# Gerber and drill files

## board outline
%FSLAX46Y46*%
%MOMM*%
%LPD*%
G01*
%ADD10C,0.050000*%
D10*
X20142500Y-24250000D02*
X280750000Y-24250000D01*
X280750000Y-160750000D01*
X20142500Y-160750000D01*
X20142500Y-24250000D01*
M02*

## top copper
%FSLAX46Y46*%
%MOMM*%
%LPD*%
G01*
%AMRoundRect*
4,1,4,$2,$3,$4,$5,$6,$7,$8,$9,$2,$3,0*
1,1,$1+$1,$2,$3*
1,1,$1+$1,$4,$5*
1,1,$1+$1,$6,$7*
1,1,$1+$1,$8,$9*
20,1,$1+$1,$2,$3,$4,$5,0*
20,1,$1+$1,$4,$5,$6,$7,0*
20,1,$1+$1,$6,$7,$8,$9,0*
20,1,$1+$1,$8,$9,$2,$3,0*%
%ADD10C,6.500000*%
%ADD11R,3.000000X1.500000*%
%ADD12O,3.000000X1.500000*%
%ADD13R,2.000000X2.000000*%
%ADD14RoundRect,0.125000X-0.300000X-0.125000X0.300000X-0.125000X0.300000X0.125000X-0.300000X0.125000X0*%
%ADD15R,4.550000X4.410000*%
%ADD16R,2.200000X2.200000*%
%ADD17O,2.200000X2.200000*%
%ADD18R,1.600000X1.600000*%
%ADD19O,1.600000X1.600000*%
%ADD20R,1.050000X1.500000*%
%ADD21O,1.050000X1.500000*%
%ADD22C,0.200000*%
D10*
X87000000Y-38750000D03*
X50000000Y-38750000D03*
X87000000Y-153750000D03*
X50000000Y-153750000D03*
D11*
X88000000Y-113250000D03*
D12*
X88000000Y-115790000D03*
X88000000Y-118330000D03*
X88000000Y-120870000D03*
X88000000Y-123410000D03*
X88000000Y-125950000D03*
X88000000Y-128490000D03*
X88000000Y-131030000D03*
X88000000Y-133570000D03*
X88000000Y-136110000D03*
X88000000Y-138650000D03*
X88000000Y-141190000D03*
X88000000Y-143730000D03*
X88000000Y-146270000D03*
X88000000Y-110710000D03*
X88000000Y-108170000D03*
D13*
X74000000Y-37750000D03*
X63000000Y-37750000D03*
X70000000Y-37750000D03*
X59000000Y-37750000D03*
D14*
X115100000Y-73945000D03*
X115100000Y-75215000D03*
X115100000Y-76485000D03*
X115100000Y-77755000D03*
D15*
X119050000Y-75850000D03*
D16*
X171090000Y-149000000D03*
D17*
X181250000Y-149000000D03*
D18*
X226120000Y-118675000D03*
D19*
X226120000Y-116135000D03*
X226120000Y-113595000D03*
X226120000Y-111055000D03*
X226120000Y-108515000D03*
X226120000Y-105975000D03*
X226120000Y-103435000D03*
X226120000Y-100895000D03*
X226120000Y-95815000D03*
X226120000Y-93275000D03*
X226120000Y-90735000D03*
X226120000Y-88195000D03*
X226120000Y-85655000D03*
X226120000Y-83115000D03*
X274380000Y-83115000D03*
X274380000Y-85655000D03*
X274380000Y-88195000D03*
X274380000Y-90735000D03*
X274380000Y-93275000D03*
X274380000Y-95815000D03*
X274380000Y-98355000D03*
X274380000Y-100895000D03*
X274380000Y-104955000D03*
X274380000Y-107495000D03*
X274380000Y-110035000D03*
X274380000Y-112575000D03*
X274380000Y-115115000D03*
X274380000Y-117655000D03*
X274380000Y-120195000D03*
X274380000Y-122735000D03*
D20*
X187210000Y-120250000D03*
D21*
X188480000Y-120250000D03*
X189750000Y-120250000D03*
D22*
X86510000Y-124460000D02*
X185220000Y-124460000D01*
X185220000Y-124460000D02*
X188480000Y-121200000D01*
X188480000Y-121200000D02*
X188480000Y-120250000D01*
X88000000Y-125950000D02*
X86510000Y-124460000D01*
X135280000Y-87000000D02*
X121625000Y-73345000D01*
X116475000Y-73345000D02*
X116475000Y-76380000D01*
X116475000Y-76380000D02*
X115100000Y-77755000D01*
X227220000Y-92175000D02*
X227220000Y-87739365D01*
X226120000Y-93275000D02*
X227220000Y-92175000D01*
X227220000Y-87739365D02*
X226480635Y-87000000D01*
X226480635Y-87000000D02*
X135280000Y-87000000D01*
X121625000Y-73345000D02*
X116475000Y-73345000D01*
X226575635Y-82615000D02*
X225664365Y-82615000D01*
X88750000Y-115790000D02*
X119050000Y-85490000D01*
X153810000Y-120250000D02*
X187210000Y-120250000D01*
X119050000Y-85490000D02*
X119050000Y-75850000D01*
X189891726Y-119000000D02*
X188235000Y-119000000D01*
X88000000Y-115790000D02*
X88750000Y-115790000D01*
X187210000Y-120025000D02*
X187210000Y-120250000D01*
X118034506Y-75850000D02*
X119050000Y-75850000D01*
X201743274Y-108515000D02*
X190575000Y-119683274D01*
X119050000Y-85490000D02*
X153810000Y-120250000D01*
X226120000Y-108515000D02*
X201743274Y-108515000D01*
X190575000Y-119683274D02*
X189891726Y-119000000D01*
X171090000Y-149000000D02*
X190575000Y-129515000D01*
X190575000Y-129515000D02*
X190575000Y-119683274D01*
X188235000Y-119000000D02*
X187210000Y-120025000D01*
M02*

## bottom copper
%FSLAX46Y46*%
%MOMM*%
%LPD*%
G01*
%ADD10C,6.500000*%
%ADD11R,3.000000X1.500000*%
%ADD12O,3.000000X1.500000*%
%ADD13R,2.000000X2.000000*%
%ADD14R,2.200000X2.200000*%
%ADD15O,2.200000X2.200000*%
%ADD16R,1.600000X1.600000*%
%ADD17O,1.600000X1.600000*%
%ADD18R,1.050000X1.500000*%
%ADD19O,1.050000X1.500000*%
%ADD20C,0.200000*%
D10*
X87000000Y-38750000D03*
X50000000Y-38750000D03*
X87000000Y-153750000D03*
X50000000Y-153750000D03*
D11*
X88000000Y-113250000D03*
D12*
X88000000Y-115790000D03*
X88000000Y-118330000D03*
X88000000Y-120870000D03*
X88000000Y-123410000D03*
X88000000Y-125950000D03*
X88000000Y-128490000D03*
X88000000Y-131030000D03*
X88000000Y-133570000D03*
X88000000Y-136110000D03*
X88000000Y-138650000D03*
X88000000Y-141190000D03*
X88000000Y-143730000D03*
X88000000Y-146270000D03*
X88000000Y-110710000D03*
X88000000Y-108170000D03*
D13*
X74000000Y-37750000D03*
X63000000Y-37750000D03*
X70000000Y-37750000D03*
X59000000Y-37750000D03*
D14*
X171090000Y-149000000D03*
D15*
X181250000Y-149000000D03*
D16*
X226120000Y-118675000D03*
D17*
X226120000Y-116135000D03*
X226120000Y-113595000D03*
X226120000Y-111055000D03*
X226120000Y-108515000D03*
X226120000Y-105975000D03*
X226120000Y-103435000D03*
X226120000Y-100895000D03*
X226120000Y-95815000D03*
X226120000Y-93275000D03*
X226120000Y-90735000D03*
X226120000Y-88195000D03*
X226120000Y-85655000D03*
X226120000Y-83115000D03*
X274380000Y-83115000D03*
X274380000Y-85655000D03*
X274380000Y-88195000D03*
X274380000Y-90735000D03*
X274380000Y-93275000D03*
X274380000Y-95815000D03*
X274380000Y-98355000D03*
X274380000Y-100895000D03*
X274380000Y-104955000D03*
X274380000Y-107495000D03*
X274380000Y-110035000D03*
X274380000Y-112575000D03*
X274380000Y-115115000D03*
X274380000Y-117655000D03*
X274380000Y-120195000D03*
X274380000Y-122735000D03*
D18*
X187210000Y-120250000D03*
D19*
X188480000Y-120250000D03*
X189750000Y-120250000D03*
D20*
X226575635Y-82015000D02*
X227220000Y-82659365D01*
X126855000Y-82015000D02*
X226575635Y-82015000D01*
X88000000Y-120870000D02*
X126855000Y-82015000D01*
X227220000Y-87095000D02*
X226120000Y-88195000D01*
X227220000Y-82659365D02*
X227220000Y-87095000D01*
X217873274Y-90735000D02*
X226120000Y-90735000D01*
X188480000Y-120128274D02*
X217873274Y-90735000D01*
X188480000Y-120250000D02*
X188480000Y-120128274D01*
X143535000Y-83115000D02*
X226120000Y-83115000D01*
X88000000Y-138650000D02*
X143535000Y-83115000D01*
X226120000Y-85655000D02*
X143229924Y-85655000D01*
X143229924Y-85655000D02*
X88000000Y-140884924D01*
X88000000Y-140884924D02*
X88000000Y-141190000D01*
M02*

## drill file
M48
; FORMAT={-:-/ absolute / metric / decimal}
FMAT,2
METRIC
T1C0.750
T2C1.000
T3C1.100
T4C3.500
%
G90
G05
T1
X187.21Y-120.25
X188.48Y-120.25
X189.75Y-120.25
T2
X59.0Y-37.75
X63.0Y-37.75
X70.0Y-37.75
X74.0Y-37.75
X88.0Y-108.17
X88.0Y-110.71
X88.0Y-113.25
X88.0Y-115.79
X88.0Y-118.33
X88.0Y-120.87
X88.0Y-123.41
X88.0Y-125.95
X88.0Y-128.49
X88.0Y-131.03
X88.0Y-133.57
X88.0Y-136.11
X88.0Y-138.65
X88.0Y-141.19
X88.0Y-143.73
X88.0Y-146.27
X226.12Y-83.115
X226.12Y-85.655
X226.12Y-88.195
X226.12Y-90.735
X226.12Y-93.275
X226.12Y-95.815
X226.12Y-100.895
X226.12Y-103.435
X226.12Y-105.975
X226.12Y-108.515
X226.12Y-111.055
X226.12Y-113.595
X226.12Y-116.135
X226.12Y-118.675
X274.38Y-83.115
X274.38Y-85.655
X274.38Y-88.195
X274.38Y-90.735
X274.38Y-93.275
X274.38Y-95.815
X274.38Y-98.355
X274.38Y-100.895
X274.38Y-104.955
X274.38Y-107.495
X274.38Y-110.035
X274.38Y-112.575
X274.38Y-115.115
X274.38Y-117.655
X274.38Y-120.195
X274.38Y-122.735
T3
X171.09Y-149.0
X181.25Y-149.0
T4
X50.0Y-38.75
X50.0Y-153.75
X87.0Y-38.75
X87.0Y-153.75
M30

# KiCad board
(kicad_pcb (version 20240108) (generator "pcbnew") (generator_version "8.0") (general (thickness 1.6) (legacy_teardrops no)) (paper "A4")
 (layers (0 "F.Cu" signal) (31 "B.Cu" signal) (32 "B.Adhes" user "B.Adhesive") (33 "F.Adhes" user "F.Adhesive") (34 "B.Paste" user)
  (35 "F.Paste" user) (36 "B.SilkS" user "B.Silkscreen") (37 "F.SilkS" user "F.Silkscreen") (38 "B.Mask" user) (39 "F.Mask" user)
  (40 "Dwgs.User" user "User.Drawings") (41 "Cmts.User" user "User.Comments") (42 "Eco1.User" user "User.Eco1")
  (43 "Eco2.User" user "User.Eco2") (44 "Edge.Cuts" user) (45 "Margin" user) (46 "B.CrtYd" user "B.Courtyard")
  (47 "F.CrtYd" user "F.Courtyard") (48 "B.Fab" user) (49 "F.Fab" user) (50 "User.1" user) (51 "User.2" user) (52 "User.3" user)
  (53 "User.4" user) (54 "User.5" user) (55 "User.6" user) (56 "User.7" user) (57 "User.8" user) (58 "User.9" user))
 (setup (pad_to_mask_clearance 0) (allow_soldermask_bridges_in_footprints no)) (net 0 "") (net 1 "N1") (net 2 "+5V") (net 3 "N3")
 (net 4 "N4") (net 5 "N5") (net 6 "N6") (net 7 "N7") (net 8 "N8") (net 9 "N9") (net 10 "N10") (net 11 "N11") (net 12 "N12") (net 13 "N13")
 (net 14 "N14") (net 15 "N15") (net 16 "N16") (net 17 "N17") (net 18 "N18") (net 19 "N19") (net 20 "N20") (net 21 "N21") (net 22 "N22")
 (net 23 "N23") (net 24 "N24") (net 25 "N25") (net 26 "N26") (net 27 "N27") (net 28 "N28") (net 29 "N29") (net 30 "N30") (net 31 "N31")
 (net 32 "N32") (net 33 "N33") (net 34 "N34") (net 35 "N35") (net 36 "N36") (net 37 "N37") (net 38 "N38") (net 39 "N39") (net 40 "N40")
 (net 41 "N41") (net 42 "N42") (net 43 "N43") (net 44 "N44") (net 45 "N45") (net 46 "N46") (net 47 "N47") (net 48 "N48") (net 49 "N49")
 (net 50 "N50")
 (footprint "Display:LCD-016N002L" (layer "F.Cu") (at 88 113.25 -90)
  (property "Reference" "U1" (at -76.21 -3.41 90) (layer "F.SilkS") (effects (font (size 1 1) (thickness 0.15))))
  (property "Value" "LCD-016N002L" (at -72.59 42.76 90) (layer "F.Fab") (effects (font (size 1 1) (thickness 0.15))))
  (pad "" thru_hole circle (at -74.5 1 90) (size 6.5 6.5) (drill 3.5) (layers "*.Cu" "*.Mask") (remove_unused_layers no))
  (pad "" thru_hole circle (at -74.5 38 90) (size 6.5 6.5) (drill 3.5) (layers "*.Cu" "*.Mask") (remove_unused_layers no))
  (pad "" thru_hole circle (at 40.5 1 90) (size 6.5 6.5) (drill 3.5) (layers "*.Cu" "*.Mask") (remove_unused_layers no))
  (pad "" thru_hole circle (at 40.5 38 90) (size 6.5 6.5) (drill 3.5) (layers "*.Cu" "*.Mask") (remove_unused_layers no))
  (pad "1" thru_hole rect (at 0 0 90) (size 1.5 3) (drill 1) (layers "*.Cu" "*.Mask") (remove_unused_layers no) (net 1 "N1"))
  (pad "2" thru_hole oval (at 2.54 0 90) (size 1.5 3) (drill 1) (layers "*.Cu" "*.Mask") (remove_unused_layers no) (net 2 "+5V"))
  (pad "3" thru_hole oval (at 5.08 0 90) (size 1.5 3) (drill 1) (layers "*.Cu" "*.Mask") (remove_unused_layers no) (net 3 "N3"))
  (pad "4" thru_hole oval (at 7.62 0 90) (size 1.5 3) (drill 1) (layers "*.Cu" "*.Mask") (remove_unused_layers no) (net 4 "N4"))
  (pad "5" thru_hole oval (at 10.16 0 90) (size 1.5 3) (drill 1) (layers "*.Cu" "*.Mask") (remove_unused_layers no) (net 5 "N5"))
  (pad "6" thru_hole oval (at 12.7 0 90) (size 1.5 3) (drill 1) (layers "*.Cu" "*.Mask") (remove_unused_layers no) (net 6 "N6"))
  (pad "7" thru_hole oval (at 15.24 0 90) (size 1.5 3) (drill 1) (layers "*.Cu" "*.Mask") (remove_unused_layers no) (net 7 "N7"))
  (pad "8" thru_hole oval (at 17.78 0 90) (size 1.5 3) (drill 1) (layers "*.Cu" "*.Mask") (remove_unused_layers no) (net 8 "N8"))
  (pad "9" thru_hole oval (at 20.32 0 90) (size 1.5 3) (drill 1) (layers "*.Cu" "*.Mask") (remove_unused_layers no) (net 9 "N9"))
  (pad "10" thru_hole oval (at 22.86 0 90) (size 1.5 3) (drill 1) (layers "*.Cu" "*.Mask") (remove_unused_layers no) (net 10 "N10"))
  (pad "11" thru_hole oval (at 25.4 0 90) (size 1.5 3) (drill 1) (layers "*.Cu" "*.Mask") (remove_unused_layers no) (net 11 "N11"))
  (pad "12" thru_hole oval (at 27.94 0 90) (size 1.5 3) (drill 1) (layers "*.Cu" "*.Mask") (remove_unused_layers no) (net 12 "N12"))
  (pad "13" thru_hole oval (at 30.48 0 90) (size 1.5 3) (drill 1) (layers "*.Cu" "*.Mask") (remove_unused_layers no) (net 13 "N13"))
  (pad "14" thru_hole oval (at 33.02 0 90) (size 1.5 3) (drill 1) (layers "*.Cu" "*.Mask") (remove_unused_layers no) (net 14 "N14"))
  (pad "15" thru_hole oval (at -2.54 0 90) (size 1.5 3) (drill 1) (layers "*.Cu" "*.Mask") (remove_unused_layers no) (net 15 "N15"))
  (pad "16" thru_hole oval (at -5.08 0 90) (size 1.5 3) (drill 1) (layers "*.Cu" "*.Mask") (remove_unused_layers no) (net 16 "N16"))
  (pad "A1" thru_hole rect (at -75.5 14 90) (size 2 2) (drill 1) (layers "*.Cu" "*.Mask") (remove_unused_layers no) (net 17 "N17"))
  (pad "A2" thru_hole rect (at -75.5 25 90) (size 2 2) (drill 1) (layers "*.Cu" "*.Mask") (remove_unused_layers no) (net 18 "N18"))
  (pad "K1" thru_hole rect (at -75.5 18 90) (size 2 2) (drill 1) (layers "*.Cu" "*.Mask") (remove_unused_layers no) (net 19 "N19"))
  (pad "K2" thru_hole rect (at -75.5 29 90) (size 2 2) (drill 1) (layers "*.Cu" "*.Mask") (remove_unused_layers no) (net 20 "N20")))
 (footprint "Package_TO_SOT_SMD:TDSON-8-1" (layer "F.Cu") (at 118 75.85)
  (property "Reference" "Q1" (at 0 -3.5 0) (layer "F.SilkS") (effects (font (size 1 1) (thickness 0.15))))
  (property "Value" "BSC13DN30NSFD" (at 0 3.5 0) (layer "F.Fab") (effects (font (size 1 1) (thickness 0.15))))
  (pad "" smd roundrect (at -0.2 -0.85) (size 1.5 1.5) (layers "F.Paste") (roundrect_rratio 0.25))
  (pad "" smd roundrect (at -0.2 0.85) (size 1.5 1.5) (layers "F.Paste") (roundrect_rratio 0.25))
  (pad "" smd custom (at 0.65 0) (size 3.75 4.41) (layers "F.Mask") (zone_connect 0) (thermal_bridge_angle 45)
   (options (clearance outline) (anchor rect)) (primitives))
  (pad "" smd roundrect (at 1.5 -0.85) (size 1.5 1.5) (layers "F.Paste") (roundrect_rratio 0.25))
  (pad "" smd roundrect (at 1.5 0.85) (size 1.5 1.5) (layers "F.Paste") (roundrect_rratio 0.25))
  (pad "" smd roundrect (at 2.905 -1.905) (size 0.75 0.5) (layers "F.Paste") (roundrect_rratio 0.25))
  (pad "" smd roundrect (at 2.905 -0.635) (size 0.75 0.5) (layers "F.Paste") (roundrect_rratio 0.25))
  (pad "" smd roundrect (at 2.905 0.635) (size 0.75 0.5) (layers "F.Paste") (roundrect_rratio 0.25))
  (pad "" smd roundrect (at 2.905 1.905) (size 0.75 0.5) (layers "F.Paste") (roundrect_rratio 0.25))
  (pad "1" smd roundrect (at -2.9 -1.905) (size 0.85 0.5) (layers "F.Cu" "F.Paste" "F.Mask") (roundrect_rratio 0.25) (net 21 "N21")
   (solder_paste_margin -0.05))
  (pad "2" smd roundrect (at -2.9 -0.635) (size 0.85 0.5) (layers "F.Cu" "F.Paste" "F.Mask") (roundrect_rratio 0.25) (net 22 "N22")
   (solder_paste_margin -0.05))
  (pad "3" smd roundrect (at -2.9 0.635) (size 0.85 0.5) (layers "F.Cu" "F.Paste" "F.Mask") (roundrect_rratio 0.25) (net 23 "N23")
   (solder_paste_margin -0.05))
  (pad "4" smd roundrect (at -2.9 1.905) (size 0.85 0.5) (layers "F.Cu" "F.Paste" "F.Mask") (roundrect_rratio 0.25) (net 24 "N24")
   (solder_paste_margin -0.05))
  (pad "5" smd rect (at 1.05 0) (size 4.55 4.41) (layers "F.Cu") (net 2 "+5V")))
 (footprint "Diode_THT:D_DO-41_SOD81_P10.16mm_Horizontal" (layer "F.Cu") (at 171.09 149)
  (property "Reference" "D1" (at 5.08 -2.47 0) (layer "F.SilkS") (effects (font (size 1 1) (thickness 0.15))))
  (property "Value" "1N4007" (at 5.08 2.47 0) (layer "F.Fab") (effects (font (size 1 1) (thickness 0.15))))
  (pad "1" thru_hole rect (at 0 0) (size 2.2 2.2) (drill 1.1) (layers "*.Cu" "*.Mask") (remove_unused_layers no) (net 2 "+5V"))
  (pad "2" thru_hole oval (at 10.16 0) (size 2.2 2.2) (drill 1.1) (layers "*.Cu" "*.Mask") (remove_unused_layers no) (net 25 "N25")))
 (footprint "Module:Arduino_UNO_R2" (layer "F.Cu") (at 226.12 118.675 90)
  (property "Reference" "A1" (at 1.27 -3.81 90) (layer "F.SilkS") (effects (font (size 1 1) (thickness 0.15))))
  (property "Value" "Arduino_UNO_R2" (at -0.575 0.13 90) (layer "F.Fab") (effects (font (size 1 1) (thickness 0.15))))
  (pad "1" thru_hole rect (at 0 0 180) (size 1.6 1.6) (drill 1) (layers "*.Cu" "*.Mask") (remove_unused_layers no) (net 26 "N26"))
  (pad "2" thru_hole oval (at 2.54 0 180) (size 1.6 1.6) (drill 1) (layers "*.Cu" "*.Mask") (remove_unused_layers no) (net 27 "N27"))
  (pad "3" thru_hole oval (at 5.08 0 180) (size 1.6 1.6) (drill 1) (layers "*.Cu" "*.Mask") (remove_unused_layers no) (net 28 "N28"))
  (pad "4" thru_hole oval (at 7.62 0 180) (size 1.6 1.6) (drill 1) (layers "*.Cu" "*.Mask") (remove_unused_layers no) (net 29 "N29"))
  (pad "5" thru_hole oval (at 10.16 0 180) (size 1.6 1.6) (drill 1) (layers "*.Cu" "*.Mask") (remove_unused_layers no) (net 2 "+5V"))
  (pad "6" thru_hole oval (at 12.7 0 180) (size 1.6 1.6) (drill 1) (layers "*.Cu" "*.Mask") (remove_unused_layers no) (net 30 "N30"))
  (pad "7" thru_hole oval (at 15.24 0 180) (size 1.6 1.6) (drill 1) (layers "*.Cu" "*.Mask") (remove_unused_layers no) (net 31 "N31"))
  (pad "8" thru_hole oval (at 17.78 0 180) (size 1.6 1.6) (drill 1) (layers "*.Cu" "*.Mask") (remove_unused_layers no) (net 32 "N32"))
  (pad "9" thru_hole oval (at 22.86 0 180) (size 1.6 1.6) (drill 1) (layers "*.Cu" "*.Mask") (remove_unused_layers no) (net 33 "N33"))
  (pad "10" thru_hole oval (at 25.4 0 180) (size 1.6 1.6) (drill 1) (layers "*.Cu" "*.Mask") (remove_unused_layers no) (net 24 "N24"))
  (pad "11" thru_hole oval (at 27.94 0 180) (size 1.6 1.6) (drill 1) (layers "*.Cu" "*.Mask") (remove_unused_layers no) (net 6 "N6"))
  (pad "12" thru_hole oval (at 30.48 0 180) (size 1.6 1.6) (drill 1) (layers "*.Cu" "*.Mask") (remove_unused_layers no) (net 4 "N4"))
  (pad "13" thru_hole oval (at 33.02 0 180) (size 1.6 1.6) (drill 1) (layers "*.Cu" "*.Mask") (remove_unused_layers no) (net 12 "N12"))
  (pad "14" thru_hole oval (at 35.56 0 180) (size 1.6 1.6) (drill 1) (layers "*.Cu" "*.Mask") (remove_unused_layers no) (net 11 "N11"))
  (pad "15" thru_hole oval (at 35.56 48.26 180) (size 1.6 1.6) (drill 1) (layers "*.Cu" "*.Mask") (remove_unused_layers no) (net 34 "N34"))
  (pad "16" thru_hole oval (at 33.02 48.26 180) (size 1.6 1.6) (drill 1) (layers "*.Cu" "*.Mask") (remove_unused_layers no) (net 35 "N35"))
  (pad "17" thru_hole oval (at 30.48 48.26 180) (size 1.6 1.6) (drill 1) (layers "*.Cu" "*.Mask") (remove_unused_layers no) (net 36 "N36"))
  (pad "18" thru_hole oval (at 27.94 48.26 180) (size 1.6 1.6) (drill 1) (layers "*.Cu" "*.Mask") (remove_unused_layers no) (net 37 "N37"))
  (pad "19" thru_hole oval (at 25.4 48.26 180) (size 1.6 1.6) (drill 1) (layers "*.Cu" "*.Mask") (remove_unused_layers no) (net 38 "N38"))
  (pad "20" thru_hole oval (at 22.86 48.26 180) (size 1.6 1.6) (drill 1) (layers "*.Cu" "*.Mask") (remove_unused_layers no) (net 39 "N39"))
  (pad "21" thru_hole oval (at 20.32 48.26 180) (size 1.6 1.6) (drill 1) (layers "*.Cu" "*.Mask") (remove_unused_layers no) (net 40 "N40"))
  (pad "22" thru_hole oval (at 17.78 48.26 180) (size 1.6 1.6) (drill 1) (layers "*.Cu" "*.Mask") (remove_unused_layers no) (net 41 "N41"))
  (pad "23" thru_hole oval (at 13.72 48.26 180) (size 1.6 1.6) (drill 1) (layers "*.Cu" "*.Mask") (remove_unused_layers no) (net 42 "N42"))
  (pad "24" thru_hole oval (at 11.18 48.26 180) (size 1.6 1.6) (drill 1) (layers "*.Cu" "*.Mask") (remove_unused_layers no) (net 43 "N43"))
  (pad "25" thru_hole oval (at 8.64 48.26 180) (size 1.6 1.6) (drill 1) (layers "*.Cu" "*.Mask") (remove_unused_layers no) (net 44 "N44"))
  (pad "26" thru_hole oval (at 6.1 48.26 180) (size 1.6 1.6) (drill 1) (layers "*.Cu" "*.Mask") (remove_unused_layers no) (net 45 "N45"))
  (pad "27" thru_hole oval (at 3.56 48.26 180) (size 1.6 1.6) (drill 1) (layers "*.Cu" "*.Mask") (remove_unused_layers no) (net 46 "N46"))
  (pad "28" thru_hole oval (at 1.02 48.26 180) (size 1.6 1.6) (drill 1) (layers "*.Cu" "*.Mask") (remove_unused_layers no) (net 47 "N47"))
  (pad "29" thru_hole oval (at -1.52 48.26 180) (size 1.6 1.6) (drill 1) (layers "*.Cu" "*.Mask") (remove_unused_layers no) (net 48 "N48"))
  (pad "30" thru_hole oval (at -4.06 48.26 180) (size 1.6 1.6) (drill 1) (layers "*.Cu" "*.Mask") (remove_unused_layers no) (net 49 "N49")))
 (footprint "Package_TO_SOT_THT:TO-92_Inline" (layer "F.Cu") (at 187.21 120.25)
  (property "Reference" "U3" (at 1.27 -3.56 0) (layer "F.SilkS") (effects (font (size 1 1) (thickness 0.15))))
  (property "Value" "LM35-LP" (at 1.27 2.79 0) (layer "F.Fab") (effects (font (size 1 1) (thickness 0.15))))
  (pad "1" thru_hole rect (at 0 0) (size 1.05 1.5) (drill 0.75) (layers "*.Cu" "*.Mask") (remove_unused_layers no) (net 2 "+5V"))
  (pad "2" thru_hole oval (at 1.27 0) (size 1.05 1.5) (drill 0.75) (layers "*.Cu" "*.Mask") (remove_unused_layers no) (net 6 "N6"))
  (pad "3" thru_hole oval (at 2.54 0) (size 1.05 1.5) (drill 0.75) (layers "*.Cu" "*.Mask") (remove_unused_layers no) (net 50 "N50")))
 (gr_rect (start 20.1425 24.25) (end 280.75 160.75) (stroke (width 0.05) (type default)) (fill none) (layer "Edge.Cuts"))
 (segment (start 226.575635 82.015) (end 227.22 82.659365) (width 0.2) (layer "B.Cu") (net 4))
 (segment (start 126.855 82.015) (end 226.575635 82.015) (width 0.2) (layer "B.Cu") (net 4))
 (segment (start 88 120.87) (end 126.855 82.015) (width 0.2) (layer "B.Cu") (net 4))
 (segment (start 227.22 87.095) (end 226.12 88.195) (width 0.2) (layer "B.Cu") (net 4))
 (segment (start 227.22 82.659365) (end 227.22 87.095) (width 0.2) (layer "B.Cu") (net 4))
 (segment (start 86.51 124.46) (end 185.22 124.46) (width 0.2) (layer "F.Cu") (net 6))
 (segment (start 185.22 124.46) (end 188.48 121.2) (width 0.2) (layer "F.Cu") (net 6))
 (segment (start 188.48 121.2) (end 188.48 120.25) (width 0.2) (layer "F.Cu") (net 6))
 (segment (start 88 125.95) (end 86.51 124.46) (width 0.2) (layer "F.Cu") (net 6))
 (segment (start 217.873274 90.735) (end 226.12 90.735) (width 0.2) (layer "B.Cu") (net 6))
 (segment (start 188.48 120.128274) (end 217.873274 90.735) (width 0.2) (layer "B.Cu") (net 6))
 (segment (start 188.48 120.25) (end 188.48 120.128274) (width 0.2) (layer "B.Cu") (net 6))
 (segment (start 135.28 87) (end 121.625 73.345) (width 0.2) (layer "F.Cu") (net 24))
 (segment (start 116.475 73.345) (end 116.475 76.38) (width 0.2) (layer "F.Cu") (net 24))
 (segment (start 116.475 76.38) (end 115.1 77.755) (width 0.2) (layer "F.Cu") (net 24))
 (segment (start 227.22 92.175) (end 227.22 87.739365) (width 0.2) (layer "F.Cu") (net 24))
 (segment (start 226.12 93.275) (end 227.22 92.175) (width 0.2) (layer "F.Cu") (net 24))
 (segment (start 227.22 87.739365) (end 226.480635 87) (width 0.2) (layer "F.Cu") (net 24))
 (segment (start 226.480635 87) (end 135.28 87) (width 0.2) (layer "F.Cu") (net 24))
 (segment (start 121.625 73.345) (end 116.475 73.345) (width 0.2) (layer "F.Cu") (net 24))
 (segment (start 226.575635 82.615) (end 225.664365 82.615) (width 0.2) (layer "F.Cu") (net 11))
 (segment (start 143.535 83.115) (end 226.12 83.115) (width 0.2) (layer "B.Cu") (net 11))
 (segment (start 88 138.65) (end 143.535 83.115) (width 0.2) (layer "B.Cu") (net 11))
 (segment (start 88.75 115.79) (end 119.05 85.49) (width 0.2) (layer "F.Cu") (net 2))
 (segment (start 153.81 120.25) (end 187.21 120.25) (width 0.2) (layer "F.Cu") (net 2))
 (segment (start 119.05 85.49) (end 119.05 75.85) (width 0.2) (layer "F.Cu") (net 2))
 (segment (start 189.891726 119) (end 188.235 119) (width 0.2) (layer "F.Cu") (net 2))
 (segment (start 88 115.79) (end 88.75 115.79) (width 0.2) (layer "F.Cu") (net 2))
 (segment (start 187.21 120.025) (end 187.21 120.25) (width 0.2) (layer "F.Cu") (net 2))
 (segment (start 118.034506 75.85) (end 119.05 75.85) (width 0.2) (layer "F.Cu") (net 2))
 (segment (start 201.743274 108.515) (end 190.575 119.683274) (width 0.2) (layer "F.Cu") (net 2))
 (segment (start 119.05 85.49) (end 153.81 120.25) (width 0.2) (layer "F.Cu") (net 2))
 (segment (start 226.12 108.515) (end 201.743274 108.515) (width 0.2) (layer "F.Cu") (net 2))
 (segment (start 190.575 119.683274) (end 189.891726 119) (width 0.2) (layer "F.Cu") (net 2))
 (segment (start 171.09 149) (end 190.575 129.515) (width 0.2) (layer "F.Cu") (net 2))
 (segment (start 190.575 129.515) (end 190.575 119.683274) (width 0.2) (layer "F.Cu") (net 2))
 (segment (start 188.235 119) (end 187.21 120.025) (width 0.2) (layer "F.Cu") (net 2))
 (segment (start 226.12 85.655) (end 143.229924 85.655) (width 0.2) (layer "B.Cu") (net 12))
 (segment (start 143.229924 85.655) (end 88 140.884924) (width 0.2) (layer "B.Cu") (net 12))
 (segment (start 88 140.884924) (end 88 141.19) (width 0.2) (layer "B.Cu") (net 12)))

